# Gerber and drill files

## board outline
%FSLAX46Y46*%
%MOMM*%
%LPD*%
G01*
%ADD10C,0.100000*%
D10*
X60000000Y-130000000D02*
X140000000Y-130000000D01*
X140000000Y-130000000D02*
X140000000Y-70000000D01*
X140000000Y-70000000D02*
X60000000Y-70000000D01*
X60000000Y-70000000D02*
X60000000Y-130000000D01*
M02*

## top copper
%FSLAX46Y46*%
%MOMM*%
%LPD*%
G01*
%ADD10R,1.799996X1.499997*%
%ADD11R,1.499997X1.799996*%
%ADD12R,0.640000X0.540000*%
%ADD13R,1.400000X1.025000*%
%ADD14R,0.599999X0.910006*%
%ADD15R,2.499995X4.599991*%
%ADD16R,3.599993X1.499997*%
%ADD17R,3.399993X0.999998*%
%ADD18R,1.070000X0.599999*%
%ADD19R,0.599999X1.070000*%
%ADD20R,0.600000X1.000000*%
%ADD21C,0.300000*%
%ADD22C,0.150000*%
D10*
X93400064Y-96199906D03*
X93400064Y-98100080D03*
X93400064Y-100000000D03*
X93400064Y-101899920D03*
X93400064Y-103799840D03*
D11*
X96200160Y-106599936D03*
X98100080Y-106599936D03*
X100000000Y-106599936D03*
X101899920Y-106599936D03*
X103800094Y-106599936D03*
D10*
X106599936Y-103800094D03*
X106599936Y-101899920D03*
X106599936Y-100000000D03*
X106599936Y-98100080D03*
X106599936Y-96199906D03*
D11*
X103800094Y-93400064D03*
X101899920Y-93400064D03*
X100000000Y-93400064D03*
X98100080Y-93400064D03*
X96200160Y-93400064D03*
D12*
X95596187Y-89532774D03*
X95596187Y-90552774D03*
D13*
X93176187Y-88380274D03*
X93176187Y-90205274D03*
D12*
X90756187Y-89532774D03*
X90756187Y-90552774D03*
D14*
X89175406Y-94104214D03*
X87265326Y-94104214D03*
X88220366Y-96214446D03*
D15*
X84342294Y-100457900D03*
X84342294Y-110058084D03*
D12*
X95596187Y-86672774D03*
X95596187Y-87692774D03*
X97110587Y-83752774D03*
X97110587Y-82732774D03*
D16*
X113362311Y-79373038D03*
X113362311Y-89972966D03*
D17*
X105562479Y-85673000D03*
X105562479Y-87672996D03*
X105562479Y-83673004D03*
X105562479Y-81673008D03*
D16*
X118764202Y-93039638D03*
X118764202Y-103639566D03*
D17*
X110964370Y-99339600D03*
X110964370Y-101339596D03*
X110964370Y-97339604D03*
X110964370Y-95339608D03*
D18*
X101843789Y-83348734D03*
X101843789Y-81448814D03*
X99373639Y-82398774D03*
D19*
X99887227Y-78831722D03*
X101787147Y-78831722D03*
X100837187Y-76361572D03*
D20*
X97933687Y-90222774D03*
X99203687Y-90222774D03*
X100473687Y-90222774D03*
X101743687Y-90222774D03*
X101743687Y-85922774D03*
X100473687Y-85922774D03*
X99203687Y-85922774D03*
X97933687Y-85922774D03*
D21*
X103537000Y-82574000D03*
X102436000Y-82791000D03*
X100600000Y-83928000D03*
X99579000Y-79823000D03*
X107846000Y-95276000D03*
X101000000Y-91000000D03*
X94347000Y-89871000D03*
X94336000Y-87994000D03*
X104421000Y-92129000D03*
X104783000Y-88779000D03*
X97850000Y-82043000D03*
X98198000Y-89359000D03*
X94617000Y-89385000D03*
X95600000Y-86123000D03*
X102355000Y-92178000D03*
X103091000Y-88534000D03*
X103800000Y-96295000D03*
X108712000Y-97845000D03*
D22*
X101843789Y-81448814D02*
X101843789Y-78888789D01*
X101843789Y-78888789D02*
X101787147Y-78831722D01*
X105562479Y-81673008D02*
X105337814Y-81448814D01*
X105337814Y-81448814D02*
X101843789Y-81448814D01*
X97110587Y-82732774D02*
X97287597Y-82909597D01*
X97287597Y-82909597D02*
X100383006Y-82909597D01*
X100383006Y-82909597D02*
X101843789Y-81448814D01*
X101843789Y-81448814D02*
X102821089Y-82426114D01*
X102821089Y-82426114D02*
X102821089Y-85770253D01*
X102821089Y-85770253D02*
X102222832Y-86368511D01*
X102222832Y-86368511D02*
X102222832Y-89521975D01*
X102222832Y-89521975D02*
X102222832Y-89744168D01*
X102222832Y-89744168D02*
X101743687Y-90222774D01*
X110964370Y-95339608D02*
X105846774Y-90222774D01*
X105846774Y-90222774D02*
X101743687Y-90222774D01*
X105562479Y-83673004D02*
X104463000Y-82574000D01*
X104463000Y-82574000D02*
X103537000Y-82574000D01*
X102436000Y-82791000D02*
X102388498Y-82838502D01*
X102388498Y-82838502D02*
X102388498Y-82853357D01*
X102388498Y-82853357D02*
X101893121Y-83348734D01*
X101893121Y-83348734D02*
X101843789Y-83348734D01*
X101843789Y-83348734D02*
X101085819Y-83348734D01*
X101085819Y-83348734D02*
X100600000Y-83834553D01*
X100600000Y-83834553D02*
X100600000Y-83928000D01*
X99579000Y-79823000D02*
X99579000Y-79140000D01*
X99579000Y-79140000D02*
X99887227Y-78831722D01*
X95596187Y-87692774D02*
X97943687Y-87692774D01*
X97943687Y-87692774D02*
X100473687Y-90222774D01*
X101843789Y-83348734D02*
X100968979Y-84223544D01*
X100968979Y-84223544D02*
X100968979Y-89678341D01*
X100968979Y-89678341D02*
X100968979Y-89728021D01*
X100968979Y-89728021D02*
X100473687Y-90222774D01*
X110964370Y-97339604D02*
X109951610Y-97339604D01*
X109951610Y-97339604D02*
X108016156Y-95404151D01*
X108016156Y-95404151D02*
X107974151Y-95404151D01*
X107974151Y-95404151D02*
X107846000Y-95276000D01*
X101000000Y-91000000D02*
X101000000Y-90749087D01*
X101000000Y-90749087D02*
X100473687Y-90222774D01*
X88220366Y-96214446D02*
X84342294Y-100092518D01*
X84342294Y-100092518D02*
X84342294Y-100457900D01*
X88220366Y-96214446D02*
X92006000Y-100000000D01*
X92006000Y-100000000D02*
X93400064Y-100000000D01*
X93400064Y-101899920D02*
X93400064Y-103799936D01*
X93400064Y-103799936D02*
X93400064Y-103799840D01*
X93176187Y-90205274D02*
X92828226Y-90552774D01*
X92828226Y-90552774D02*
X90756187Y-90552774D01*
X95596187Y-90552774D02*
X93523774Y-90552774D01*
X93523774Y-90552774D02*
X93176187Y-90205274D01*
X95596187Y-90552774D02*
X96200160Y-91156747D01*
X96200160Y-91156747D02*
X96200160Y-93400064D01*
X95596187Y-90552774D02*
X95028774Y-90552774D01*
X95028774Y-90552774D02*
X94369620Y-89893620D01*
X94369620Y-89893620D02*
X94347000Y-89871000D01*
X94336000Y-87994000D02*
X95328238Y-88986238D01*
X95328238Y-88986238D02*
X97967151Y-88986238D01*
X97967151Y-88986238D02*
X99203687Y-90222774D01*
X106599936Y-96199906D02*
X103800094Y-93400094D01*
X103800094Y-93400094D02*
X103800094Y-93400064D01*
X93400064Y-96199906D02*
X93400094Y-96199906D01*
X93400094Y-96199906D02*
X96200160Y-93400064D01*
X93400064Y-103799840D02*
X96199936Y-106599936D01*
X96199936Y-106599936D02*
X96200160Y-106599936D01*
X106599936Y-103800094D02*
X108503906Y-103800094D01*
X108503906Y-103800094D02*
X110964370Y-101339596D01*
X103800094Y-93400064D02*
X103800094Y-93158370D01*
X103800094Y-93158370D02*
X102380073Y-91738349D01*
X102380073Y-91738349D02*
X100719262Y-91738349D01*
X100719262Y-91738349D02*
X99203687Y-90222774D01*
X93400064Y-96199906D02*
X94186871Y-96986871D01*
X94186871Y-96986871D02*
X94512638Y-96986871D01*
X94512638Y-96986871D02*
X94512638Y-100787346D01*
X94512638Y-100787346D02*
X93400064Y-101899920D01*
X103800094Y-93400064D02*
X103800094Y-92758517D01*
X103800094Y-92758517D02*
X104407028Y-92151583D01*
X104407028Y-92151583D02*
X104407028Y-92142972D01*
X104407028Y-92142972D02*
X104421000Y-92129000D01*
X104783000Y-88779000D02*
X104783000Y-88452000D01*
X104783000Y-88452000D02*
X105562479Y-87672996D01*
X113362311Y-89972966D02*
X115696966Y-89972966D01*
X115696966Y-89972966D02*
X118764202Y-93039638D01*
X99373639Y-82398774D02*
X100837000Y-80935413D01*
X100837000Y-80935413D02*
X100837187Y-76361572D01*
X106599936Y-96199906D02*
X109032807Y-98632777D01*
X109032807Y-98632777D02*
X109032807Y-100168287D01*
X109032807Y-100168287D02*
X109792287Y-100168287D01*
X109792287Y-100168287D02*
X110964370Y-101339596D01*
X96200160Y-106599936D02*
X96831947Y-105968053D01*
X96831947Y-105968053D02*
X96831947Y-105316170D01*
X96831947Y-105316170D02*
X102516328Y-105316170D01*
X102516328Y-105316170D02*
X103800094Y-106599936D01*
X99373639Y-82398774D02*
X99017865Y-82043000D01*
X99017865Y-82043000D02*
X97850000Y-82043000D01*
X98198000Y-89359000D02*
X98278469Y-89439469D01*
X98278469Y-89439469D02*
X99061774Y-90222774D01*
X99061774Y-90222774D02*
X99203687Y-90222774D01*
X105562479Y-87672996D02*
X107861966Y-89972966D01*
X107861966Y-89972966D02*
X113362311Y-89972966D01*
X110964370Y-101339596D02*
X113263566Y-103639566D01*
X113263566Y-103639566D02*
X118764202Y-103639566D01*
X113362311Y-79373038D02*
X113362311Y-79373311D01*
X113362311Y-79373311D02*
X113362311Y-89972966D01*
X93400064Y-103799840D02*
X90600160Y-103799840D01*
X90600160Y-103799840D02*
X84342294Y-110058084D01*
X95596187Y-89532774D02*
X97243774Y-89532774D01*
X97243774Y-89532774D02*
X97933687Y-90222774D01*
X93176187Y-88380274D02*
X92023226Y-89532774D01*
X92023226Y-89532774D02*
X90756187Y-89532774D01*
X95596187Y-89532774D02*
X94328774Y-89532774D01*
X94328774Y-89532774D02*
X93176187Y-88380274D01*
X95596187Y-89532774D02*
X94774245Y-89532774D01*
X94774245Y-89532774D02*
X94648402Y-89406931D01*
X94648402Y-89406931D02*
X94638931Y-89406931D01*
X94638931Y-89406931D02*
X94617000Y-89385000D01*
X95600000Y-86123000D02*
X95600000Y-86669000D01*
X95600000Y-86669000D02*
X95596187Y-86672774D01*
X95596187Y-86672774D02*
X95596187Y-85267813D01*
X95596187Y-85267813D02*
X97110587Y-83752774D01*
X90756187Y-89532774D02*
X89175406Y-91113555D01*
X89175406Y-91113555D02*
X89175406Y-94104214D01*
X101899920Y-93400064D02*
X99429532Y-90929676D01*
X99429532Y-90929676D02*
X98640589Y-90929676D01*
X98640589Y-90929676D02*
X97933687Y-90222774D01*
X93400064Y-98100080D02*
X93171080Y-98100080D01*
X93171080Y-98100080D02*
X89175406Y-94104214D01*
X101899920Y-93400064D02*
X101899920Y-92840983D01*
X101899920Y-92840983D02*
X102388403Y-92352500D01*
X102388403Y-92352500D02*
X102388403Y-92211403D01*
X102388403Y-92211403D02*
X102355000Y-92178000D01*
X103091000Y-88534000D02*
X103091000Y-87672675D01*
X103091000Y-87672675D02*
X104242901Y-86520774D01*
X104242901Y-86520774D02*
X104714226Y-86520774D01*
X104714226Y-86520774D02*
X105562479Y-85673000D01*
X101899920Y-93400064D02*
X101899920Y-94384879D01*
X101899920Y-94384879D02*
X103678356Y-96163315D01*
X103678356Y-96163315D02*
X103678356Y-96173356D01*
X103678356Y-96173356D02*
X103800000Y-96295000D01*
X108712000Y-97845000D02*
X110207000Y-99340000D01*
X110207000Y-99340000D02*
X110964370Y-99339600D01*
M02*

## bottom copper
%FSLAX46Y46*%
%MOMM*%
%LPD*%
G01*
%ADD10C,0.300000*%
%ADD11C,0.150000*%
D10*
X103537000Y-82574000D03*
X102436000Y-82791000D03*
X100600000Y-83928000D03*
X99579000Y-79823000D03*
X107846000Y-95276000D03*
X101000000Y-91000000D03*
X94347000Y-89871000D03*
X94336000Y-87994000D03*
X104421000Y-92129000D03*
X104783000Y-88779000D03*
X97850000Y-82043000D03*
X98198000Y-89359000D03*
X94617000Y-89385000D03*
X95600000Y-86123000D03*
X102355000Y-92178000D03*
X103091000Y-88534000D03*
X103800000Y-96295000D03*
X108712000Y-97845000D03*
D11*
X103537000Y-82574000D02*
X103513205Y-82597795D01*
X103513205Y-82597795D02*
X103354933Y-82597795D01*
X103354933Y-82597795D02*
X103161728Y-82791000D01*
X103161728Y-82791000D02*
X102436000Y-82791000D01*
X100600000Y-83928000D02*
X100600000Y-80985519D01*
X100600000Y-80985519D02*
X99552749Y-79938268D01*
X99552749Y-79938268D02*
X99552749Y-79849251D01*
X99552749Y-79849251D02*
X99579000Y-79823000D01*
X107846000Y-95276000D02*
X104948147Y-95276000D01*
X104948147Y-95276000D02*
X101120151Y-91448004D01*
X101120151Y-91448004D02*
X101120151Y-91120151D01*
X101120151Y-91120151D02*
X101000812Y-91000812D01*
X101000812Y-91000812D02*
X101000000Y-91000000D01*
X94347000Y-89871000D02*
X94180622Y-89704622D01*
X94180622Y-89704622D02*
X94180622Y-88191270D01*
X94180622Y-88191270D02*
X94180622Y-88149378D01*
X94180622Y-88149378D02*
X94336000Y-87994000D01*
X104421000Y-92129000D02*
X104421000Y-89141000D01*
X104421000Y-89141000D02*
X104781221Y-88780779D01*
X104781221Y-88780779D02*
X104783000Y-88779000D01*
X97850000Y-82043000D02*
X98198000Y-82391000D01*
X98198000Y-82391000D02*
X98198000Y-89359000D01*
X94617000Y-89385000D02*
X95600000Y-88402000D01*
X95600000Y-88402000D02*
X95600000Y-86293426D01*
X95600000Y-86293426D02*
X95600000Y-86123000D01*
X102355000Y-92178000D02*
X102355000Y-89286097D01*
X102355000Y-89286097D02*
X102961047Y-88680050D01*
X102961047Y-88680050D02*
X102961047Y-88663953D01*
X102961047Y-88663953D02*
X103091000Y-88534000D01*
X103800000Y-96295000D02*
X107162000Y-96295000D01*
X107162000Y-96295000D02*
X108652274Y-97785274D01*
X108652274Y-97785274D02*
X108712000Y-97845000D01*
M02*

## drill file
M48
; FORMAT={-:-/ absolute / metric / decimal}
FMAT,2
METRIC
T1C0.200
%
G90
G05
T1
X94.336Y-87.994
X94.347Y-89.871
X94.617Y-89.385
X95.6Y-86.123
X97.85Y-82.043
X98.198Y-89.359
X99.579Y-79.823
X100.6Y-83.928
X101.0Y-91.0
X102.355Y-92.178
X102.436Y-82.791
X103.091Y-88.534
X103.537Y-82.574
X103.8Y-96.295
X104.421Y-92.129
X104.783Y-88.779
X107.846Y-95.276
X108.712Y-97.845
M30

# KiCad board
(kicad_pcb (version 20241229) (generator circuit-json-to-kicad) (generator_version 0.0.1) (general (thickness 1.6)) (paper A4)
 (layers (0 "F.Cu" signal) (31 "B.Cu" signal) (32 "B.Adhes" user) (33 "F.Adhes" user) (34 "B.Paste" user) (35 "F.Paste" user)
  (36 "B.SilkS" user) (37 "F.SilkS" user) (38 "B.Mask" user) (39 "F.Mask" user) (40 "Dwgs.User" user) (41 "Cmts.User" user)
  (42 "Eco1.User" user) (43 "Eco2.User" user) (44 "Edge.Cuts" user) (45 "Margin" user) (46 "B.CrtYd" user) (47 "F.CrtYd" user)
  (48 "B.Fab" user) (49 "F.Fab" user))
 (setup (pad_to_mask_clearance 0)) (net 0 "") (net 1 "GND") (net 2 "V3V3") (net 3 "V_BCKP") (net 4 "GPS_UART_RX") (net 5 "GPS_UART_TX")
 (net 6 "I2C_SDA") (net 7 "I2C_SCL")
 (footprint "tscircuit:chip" (layer F.Cu) (at 100 100 0)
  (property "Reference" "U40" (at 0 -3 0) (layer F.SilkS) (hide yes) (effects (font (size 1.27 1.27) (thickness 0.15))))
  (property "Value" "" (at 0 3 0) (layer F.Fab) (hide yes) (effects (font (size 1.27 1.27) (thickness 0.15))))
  (pad "1" smd rect (at -6.5999360000001275 -3.8000939999998877 0) (size 1.7999964 1.499997) (layers F.Cu F.Paste F.Mask) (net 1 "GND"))
  (pad "2" smd rect (at -6.5999360000001275 -1.899919999999895 0) (size 1.7999964 1.499997) (layers F.Cu F.Paste F.Mask) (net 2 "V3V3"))
  (pad "3" smd rect (at -6.5999360000001275 5.684341886080802e-14 0) (size 1.7999964 1.499997) (layers F.Cu F.Paste F.Mask) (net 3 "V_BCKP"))
  (pad "4" smd rect (at -6.5999360000001275 1.8999200000000087 0) (size 1.7999964 1.499997) (layers F.Cu F.Paste F.Mask) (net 1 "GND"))
  (pad "5" smd rect (at -6.5999360000001275 3.7998400000000743 0) (size 1.7999964 1.499997) (layers F.Cu F.Paste F.Mask) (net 1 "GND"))
  (pad "6" smd rect (at -3.7998399999999606 6.599936000000014 0) (size 1.499997 1.7999964) (layers F.Cu F.Paste F.Mask) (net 1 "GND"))
  (pad "7" smd rect (at -1.899919999999895 6.599936000000014 0) (size 1.499997 1.7999964) (layers F.Cu F.Paste F.Mask))
  (pad "8" smd rect (at -5.684341886080802e-14 6.599936000000014 0) (size 1.499997 1.7999964) (layers F.Cu F.Paste F.Mask))
  (pad "9" smd rect (at 1.899919999999895 6.599936000000014 0) (size 1.499997 1.7999964) (layers F.Cu F.Paste F.Mask))
  (pad "10" smd rect (at 3.8000940000000014 6.599936000000014 0) (size 1.499997 1.7999964) (layers F.Cu F.Paste F.Mask) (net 1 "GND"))
  (pad "11" smd rect (at 6.5999360000001275 3.800094000000115 0) (size 1.7999964 1.499997) (layers F.Cu F.Paste F.Mask) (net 1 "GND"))
  (pad "12" smd rect (at 6.5999360000001275 1.8999200000000087 0) (size 1.7999964 1.499997) (layers F.Cu F.Paste F.Mask))
  (pad "13" smd rect (at 6.5999360000001275 5.684341886080802e-14 0) (size 1.7999964 1.499997) (layers F.Cu F.Paste F.Mask)
   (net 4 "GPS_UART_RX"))
  (pad "14" smd rect (at 6.5999360000001275 -1.899919999999895 0) (size 1.7999964 1.499997) (layers F.Cu F.Paste F.Mask)
   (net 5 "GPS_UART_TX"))
  (pad "15" smd rect (at 6.5999360000001275 -3.8000939999998877 0) (size 1.7999964 1.499997) (layers F.Cu F.Paste F.Mask) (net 1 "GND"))
  (pad "16" smd rect (at 3.8000940000000014 -6.599936000000014 0) (size 1.499997 1.7999964) (layers F.Cu F.Paste F.Mask) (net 1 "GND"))
  (pad "17" smd rect (at 1.899919999999895 -6.599936000000014 0) (size 1.499997 1.7999964) (layers F.Cu F.Paste F.Mask) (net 2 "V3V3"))
  (pad "18" smd rect (at -5.684341886080802e-14 -6.599936000000014 0) (size 1.499997 1.7999964) (layers F.Cu F.Paste F.Mask))
  (pad "19" smd rect (at -1.899919999999895 -6.599936000000014 0) (size 1.499997 1.7999964) (layers F.Cu F.Paste F.Mask))
  (pad "20" smd rect (at -3.7998399999999606 -6.599936000000014 0) (size 1.499997 1.7999964) (layers F.Cu F.Paste F.Mask) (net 1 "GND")))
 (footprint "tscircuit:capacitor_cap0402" (layer F.Cu) (at 95.59618690909089 90.04277400000001 -90.00000000000001)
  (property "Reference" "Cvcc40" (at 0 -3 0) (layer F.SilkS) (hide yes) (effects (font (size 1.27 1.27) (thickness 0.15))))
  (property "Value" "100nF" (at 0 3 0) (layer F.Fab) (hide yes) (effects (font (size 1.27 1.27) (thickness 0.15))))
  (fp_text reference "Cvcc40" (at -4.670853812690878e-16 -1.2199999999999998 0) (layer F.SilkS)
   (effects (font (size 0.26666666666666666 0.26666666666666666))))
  (pad "1" smd rect (at -0.5099999999999998 8.881784197001252e-16 0) (size 0.64 0.54) (layers F.Cu F.Paste F.Mask) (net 2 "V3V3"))
  (pad "2" smd rect (at 0.5099999999999998 0 0) (size 0.64 0.54) (layers F.Cu F.Paste F.Mask) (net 1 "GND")))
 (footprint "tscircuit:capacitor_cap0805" (layer F.Cu) (at 93.17618690909089 89.29277400000001 -90.00000000000001)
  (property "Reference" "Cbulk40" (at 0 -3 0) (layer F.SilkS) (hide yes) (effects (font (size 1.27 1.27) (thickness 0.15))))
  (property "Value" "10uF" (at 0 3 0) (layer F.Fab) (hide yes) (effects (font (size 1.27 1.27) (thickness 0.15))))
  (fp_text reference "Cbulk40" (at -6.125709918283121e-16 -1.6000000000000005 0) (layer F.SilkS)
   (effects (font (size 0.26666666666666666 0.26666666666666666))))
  (pad "1" smd rect (at -0.9124999999999996 0 0) (size 1.4 1.025) (layers F.Cu F.Paste F.Mask) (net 2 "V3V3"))
  (pad "2" smd rect (at 0.9124999999999996 -8.881784197001252e-16 0) (size 1.4 1.025) (layers F.Cu F.Paste F.Mask) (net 1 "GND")))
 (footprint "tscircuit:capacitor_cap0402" (layer F.Cu) (at 90.75618690909089 90.04277400000001 -90.00000000000001)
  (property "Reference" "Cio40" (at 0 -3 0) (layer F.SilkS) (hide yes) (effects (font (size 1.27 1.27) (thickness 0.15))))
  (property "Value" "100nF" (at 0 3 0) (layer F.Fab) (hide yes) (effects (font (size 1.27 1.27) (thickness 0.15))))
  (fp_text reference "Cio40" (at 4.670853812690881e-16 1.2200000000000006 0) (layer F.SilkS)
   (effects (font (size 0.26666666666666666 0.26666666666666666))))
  (pad "1" smd rect (at -0.5099999999999998 0 0) (size 0.64 0.54) (layers F.Cu F.Paste F.Mask) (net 2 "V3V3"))
  (pad "2" smd rect (at 0.5099999999999998 0 0) (size 0.64 0.54) (layers F.Cu F.Paste F.Mask) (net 1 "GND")))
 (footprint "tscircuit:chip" (layer F.Cu) (at 88.22036600000001 95.15933033333334 90)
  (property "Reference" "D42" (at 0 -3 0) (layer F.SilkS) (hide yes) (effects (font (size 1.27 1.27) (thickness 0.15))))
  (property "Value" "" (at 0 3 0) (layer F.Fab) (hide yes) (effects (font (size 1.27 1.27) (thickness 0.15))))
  (pad "1" smd rect (at 1.0551160000000053 0.9550400000000039 0) (size 0.5999987999999999 0.9100057999999999) (layers F.Cu F.Paste F.Mask)
   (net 2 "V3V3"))
  (pad "2" smd rect (at 1.0551160000000053 -0.9550400000000039 0) (size 0.5999987999999999 0.9100057999999999) (layers F.Cu F.Paste F.Mask))
  (pad "3" smd rect (at -1.0551160000000053 7.105427357601002e-15 0) (size 0.5999987999999999 0.9100057999999999)
   (layers F.Cu F.Paste F.Mask) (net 3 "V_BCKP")))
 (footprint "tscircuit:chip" (layer F.Cu) (at 84.34229399999987 105.25799233333349 -90.00000000000001)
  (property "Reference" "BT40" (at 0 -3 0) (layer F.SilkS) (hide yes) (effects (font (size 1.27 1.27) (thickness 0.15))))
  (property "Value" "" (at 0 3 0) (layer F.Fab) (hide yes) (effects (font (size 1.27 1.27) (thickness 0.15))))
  (pad "1" smd rect (at -4.80009200000012 1.7763568394002505e-15 0) (size 2.4999949999999997 4.5999908) (layers F.Cu F.Paste F.Mask)
   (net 3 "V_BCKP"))
  (pad "2" smd rect (at 4.800092000000118 -1.7763568394002505e-15 0) (size 2.4999949999999997 4.5999908) (layers F.Cu F.Paste F.Mask)
   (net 1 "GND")))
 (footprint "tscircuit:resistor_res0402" (layer F.Cu) (at 95.59618690909089 87.18277400000002 -90.00000000000001)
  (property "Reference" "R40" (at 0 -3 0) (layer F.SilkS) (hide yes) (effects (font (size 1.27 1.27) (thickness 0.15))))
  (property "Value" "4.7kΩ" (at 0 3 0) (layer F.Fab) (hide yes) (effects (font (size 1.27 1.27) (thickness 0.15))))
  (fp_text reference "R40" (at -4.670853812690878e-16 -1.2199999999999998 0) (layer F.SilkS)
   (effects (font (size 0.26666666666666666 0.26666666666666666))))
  (pad "1" smd rect (at -0.5099999999999998 0 0) (size 0.64 0.54) (layers F.Cu F.Paste F.Mask) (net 2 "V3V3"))
  (pad "2" smd rect (at 0.5099999999999998 -8.881784197001252e-16 0) (size 0.64 0.54) (layers F.Cu F.Paste F.Mask) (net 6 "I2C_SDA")))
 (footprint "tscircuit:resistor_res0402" (layer F.Cu) (at 97.11058690909073 83.24277400000001 90)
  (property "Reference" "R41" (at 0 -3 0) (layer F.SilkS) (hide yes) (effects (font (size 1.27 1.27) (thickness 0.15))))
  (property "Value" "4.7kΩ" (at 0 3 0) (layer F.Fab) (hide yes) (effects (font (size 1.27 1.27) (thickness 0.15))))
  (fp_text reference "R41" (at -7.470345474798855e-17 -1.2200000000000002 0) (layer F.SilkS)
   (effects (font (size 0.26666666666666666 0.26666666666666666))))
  (pad "1" smd rect (at -0.5100000000000016 0 0) (size 0.64 0.54) (layers F.Cu F.Paste F.Mask) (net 2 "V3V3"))
  (pad "2" smd rect (at 0.5100000000000016 0 0) (size 0.64 0.54) (layers F.Cu F.Paste F.Mask) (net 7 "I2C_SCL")))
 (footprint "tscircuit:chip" (layer F.Cu) (at 109.51239480909098 84.673002 90)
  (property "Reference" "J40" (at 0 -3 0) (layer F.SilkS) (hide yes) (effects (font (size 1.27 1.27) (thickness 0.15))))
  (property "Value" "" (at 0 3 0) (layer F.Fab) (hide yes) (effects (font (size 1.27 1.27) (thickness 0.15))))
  (pad "5" smd rect (at 5.299963999999989 3.8499161000000193 0) (size 3.5999928 1.499997) (layers F.Cu F.Paste F.Mask) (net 1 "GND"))
  (pad "6" smd rect (at -5.299963999999989 3.849916100000021 0) (size 3.5999928 1.499997) (layers F.Cu F.Paste F.Mask) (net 1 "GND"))
  (pad "2" smd rect (at -0.9999979999999482 -3.9499159000000175 0) (size 3.3999932 0.9999979999999999) (layers F.Cu F.Paste F.Mask)
   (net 2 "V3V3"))
  (pad "1" smd rect (at -2.999994000000072 -3.9499159000000175 0) (size 3.3999932 0.9999979999999999) (layers F.Cu F.Paste F.Mask)
   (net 1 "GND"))
  (pad "3" smd rect (at 0.9999979999999482 -3.9499159000000175 0) (size 3.3999932 0.9999979999999999) (layers F.Cu F.Paste F.Mask)
   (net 6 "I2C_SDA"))
  (pad "4" smd rect (at 2.9999939999999583 -3.9499159000000175 0) (size 3.3999932 0.9999979999999999) (layers F.Cu F.Paste F.Mask)
   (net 7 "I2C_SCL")))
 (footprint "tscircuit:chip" (layer F.Cu) (at 114.9142860999999 98.33960200000001 90)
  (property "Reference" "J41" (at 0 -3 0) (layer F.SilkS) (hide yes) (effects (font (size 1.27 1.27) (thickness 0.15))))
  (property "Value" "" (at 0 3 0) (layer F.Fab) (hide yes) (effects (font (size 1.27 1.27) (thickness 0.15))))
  (pad "5" smd rect (at 5.299963999999989 3.8499161000000193 0) (size 3.5999928 1.499997) (layers F.Cu F.Paste F.Mask) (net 1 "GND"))
  (pad "6" smd rect (at -5.299963999999989 3.8499161000000193 0) (size 3.5999928 1.499997) (layers F.Cu F.Paste F.Mask) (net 1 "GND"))
  (pad "2" smd rect (at -0.9999979999999482 -3.9499159000000184 0) (size 3.3999932 0.9999979999999999) (layers F.Cu F.Paste F.Mask)
   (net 2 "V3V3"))
  (pad "1" smd rect (at -2.999994000000072 -3.9499159000000184 0) (size 3.3999932 0.9999979999999999) (layers F.Cu F.Paste F.Mask)
   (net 1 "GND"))
  (pad "3" smd rect (at 0.9999979999999482 -3.9499159000000184 0) (size 3.3999932 0.9999979999999999) (layers F.Cu F.Paste F.Mask)
   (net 6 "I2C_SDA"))
  (pad "4" smd rect (at 2.9999939999999583 -3.9499159000000184 0) (size 3.3999932 0.9999979999999999) (layers F.Cu F.Paste F.Mask)
   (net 7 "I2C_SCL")))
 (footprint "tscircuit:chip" (layer F.Cu) (at 100.60871390909071 82.39877400000002 0)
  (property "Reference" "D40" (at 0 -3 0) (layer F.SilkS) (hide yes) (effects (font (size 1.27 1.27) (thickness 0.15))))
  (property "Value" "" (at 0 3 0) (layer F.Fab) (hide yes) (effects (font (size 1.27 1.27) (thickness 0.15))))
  (pad "1" smd rect (at 1.2350749999999948 0.9499599999999191 0) (size 1.0700004 0.5999987999999999) (layers F.Cu F.Paste F.Mask)
   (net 6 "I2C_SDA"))
  (pad "2" smd rect (at 1.2350749999999948 -0.9499599999999191 0) (size 1.0700004 0.5999987999999999) (layers F.Cu F.Paste F.Mask)
   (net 7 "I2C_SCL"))
  (pad "3" smd rect (at -1.2350749999999948 0 0) (size 1.0700004 0.5999987999999999) (layers F.Cu F.Paste F.Mask) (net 1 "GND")))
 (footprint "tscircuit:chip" (layer F.Cu) (at 100.83718690909089 77.59664700000003 -90.00000000000001)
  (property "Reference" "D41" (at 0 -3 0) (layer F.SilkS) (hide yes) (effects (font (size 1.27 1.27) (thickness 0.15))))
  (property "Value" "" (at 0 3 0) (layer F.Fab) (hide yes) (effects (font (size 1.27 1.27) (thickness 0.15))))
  (pad "1" smd rect (at 1.2350749999999948 0.9499599999999189 0) (size 0.5999987999999999 1.0700004) (layers F.Cu F.Paste F.Mask)
   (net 6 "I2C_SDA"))
  (pad "2" smd rect (at 1.2350749999999948 -0.9499599999999194 0) (size 0.5999987999999999 1.0700004) (layers F.Cu F.Paste F.Mask)
   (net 7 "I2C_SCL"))
  (pad "3" smd rect (at -1.2350749999999948 3.3306690738754696e-16 0) (size 0.5999987999999999 1.0700004) (layers F.Cu F.Paste F.Mask)
   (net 1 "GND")))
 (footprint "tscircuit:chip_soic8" (layer F.Cu) (at 99.83868690909088 88.07277400000001 90)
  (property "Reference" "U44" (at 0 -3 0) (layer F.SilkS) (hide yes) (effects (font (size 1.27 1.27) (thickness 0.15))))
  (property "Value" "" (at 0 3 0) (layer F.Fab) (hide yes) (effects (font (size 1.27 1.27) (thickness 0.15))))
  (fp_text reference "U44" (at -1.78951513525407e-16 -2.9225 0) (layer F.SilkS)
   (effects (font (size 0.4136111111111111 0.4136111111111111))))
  (pad "1" smd rect (at -2.1500000000000004 -1.905 0) (size 0.6 1) (layers F.Cu F.Paste F.Mask) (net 2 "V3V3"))
  (pad "2" smd rect (at -2.1500000000000004 -0.635 0) (size 0.6 1) (layers F.Cu F.Paste F.Mask) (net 1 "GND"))
  (pad "3" smd rect (at -2.1500000000000004 0.635 0) (size 0.6 1) (layers F.Cu F.Paste F.Mask) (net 6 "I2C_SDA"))
  (pad "4" smd rect (at -2.1500000000000004 1.9049999999999998 0) (size 0.6 1) (layers F.Cu F.Paste F.Mask) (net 7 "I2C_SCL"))
  (pad "5" smd rect (at 2.1500000000000004 1.905 0) (size 0.6 1) (layers F.Cu F.Paste F.Mask))
  (pad "6" smd rect (at 2.1500000000000004 0.635 0) (size 0.6 1) (layers F.Cu F.Paste F.Mask))
  (pad "7" smd rect (at 2.1500000000000004 -0.635 0) (size 0.6 1) (layers F.Cu F.Paste F.Mask))
  (pad "8" smd rect (at 2.1500000000000004 -1.905 0) (size 0.6 1) (layers F.Cu F.Paste F.Mask)))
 (segment (start 101.8437889090907 81.4488140000001) (end 101.8437889090907 78.8887889090907) (width 0.15) (layer F.Cu) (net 7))
 (segment (start 101.8437889090907 78.8887889090907) (end 101.78714690909081 78.83172200000003) (width 0.15) (layer F.Cu) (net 7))
 (segment (start 105.56247890909097 81.67300800000004) (end 105.3378140000001 81.4488140000001) (width 0.15) (layer F.Cu) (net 7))
 (segment (start 105.3378140000001 81.4488140000001) (end 101.8437889090907 81.4488140000001) (width 0.15) (layer F.Cu) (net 7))
 (segment (start 97.11058690909073 82.732774) (end 97.28759723607489 82.90959723607489) (width 0.15) (layer F.Cu) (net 7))
 (segment (start 97.28759723607489 82.90959723607489) (end 100.3830056730159 82.90959723607489) (width 0.15) (layer F.Cu) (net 7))
 (segment (start 100.3830056730159 82.90959723607489) (end 101.8437889090907 81.4488140000001) (width 0.15) (layer F.Cu) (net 7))
 (segment (start 101.8437889090907 81.4488140000001) (end 102.82108920157091 82.4261142924803) (width 0.15) (layer F.Cu) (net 7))
 (segment (start 102.82108920157091 82.4261142924803) (end 102.82108920157091 85.77025333037076) (width 0.15) (layer F.Cu) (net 7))
 (segment (start 102.82108920157091 85.77025333037076) (end 102.22283199472146 86.3685105372202) (width 0.15) (layer F.Cu) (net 7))
 (segment (start 102.22283199472146 86.3685105372202) (end 102.22283199472146 89.52197478346525) (width 0.15) (layer F.Cu) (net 7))
 (segment (start 102.22283199472146 89.52197478346525) (end 102.22283199472146 89.74416800527854) (width 0.15) (layer F.Cu) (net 7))
 (segment (start 102.22283199472146 89.74416800527854) (end 101.74368690909088 90.22277400000002) (width 0.15) (layer F.Cu) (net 7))
 (segment (start 110.96437019999988 95.33960800000006) (end 105.84677400000001 90.22277400000002) (width 0.15) (layer F.Cu) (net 7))
 (segment (start 105.84677400000001 90.22277400000002) (end 101.74368690909088 90.22277400000002) (width 0.15) (layer F.Cu) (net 7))
 (segment (start 105.56247890909097 83.67300400000005) (end 104.46300000000001 82.574) (width 0.15) (layer F.Cu) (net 6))
 (segment (start 104.46300000000001 82.574) (end 103.537 82.574) (width 0.15) (layer F.Cu) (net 6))
 (segment (start 103.537 82.574) (end 103.51320467501183 82.59779532498817) (width 0.15) (layer B.Cu) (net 6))
 (segment (start 103.51320467501183 82.59779532498817) (end 103.35493272030583 82.59779532498817) (width 0.15) (layer B.Cu) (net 6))
 (segment (start 103.35493272030583 82.59779532498817) (end 103.161728045294 82.791) (width 0.15) (layer B.Cu) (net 6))
 (segment (start 103.161728045294 82.791) (end 102.436 82.791) (width 0.15) (layer B.Cu) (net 6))
 (segment (start 102.436 82.791) (end 102.38849819781895 82.83850180218104) (width 0.15) (layer F.Cu) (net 6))
 (segment (start 102.38849819781895 82.83850180218104) (end 102.38849819781895 82.85335684220804) (width 0.15) (layer F.Cu) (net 6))
 (segment (start 102.38849819781895 82.85335684220804) (end 101.89312104002707 83.34873399999994) (width 0.15) (layer F.Cu) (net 6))
 (segment (start 101.89312104002707 83.34873399999994) (end 101.8437889090907 83.34873399999994) (width 0.15) (layer F.Cu) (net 6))
 (segment (start 101.8437889090907 83.34873399999994) (end 101.08581889302985 83.34873399999994) (width 0.15) (layer F.Cu) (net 6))
 (segment (start 101.08581889302985 83.34873399999994) (end 100.6 83.8345528930298) (width 0.15) (layer F.Cu) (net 6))
 (segment (start 100.6 83.8345528930298) (end 100.6 83.928) (width 0.15) (layer F.Cu) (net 6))
 (segment (start 100.6 83.928) (end 100.6 80.98551869050203) (width 0.15) (layer B.Cu) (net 6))
 (segment (start 100.6 80.98551869050203) (end 99.55274927718217 79.9382679676842) (width 0.15) (layer B.Cu) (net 6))
 (segment (start 99.55274927718217 79.9382679676842) (end 99.55274927718217 79.84925072281783) (width 0.15) (layer B.Cu) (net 6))
 (segment (start 99.55274927718217 79.84925072281783) (end 99.579 79.82300000000001) (width 0.15) (layer B.Cu) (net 6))
 (segment (start 99.579 79.82300000000001) (end 99.579 79.14) (width 0.15) (layer F.Cu) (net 6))
 (segment (start 99.579 79.14) (end 99.88722690909097 78.83172200000003) (width 0.15) (layer F.Cu) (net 6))
 (segment (start 95.59618690909089 87.69277400000001) (end 97.94368690909089 87.69277400000001) (width 0.15) (layer F.Cu) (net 6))
 (segment (start 97.94368690909089 87.69277400000001) (end 100.47368690909089 90.22277400000002) (width 0.15) (layer F.Cu) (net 6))
 (segment (start 101.8437889090907 83.34873399999994) (end 100.96897882086891 84.22354408822173) (width 0.15) (layer F.Cu) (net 6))
 (segment (start 100.96897882086891 84.22354408822173) (end 100.96897882086891 89.6783406450725) (width 0.15) (layer F.Cu) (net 6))
 (segment (start 100.96897882086891 89.6783406450725) (end 100.96897882086891 89.72802117913109) (width 0.15) (layer F.Cu) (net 6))
 (segment (start 100.96897882086891 89.72802117913109) (end 100.47368690909089 90.22277400000002) (width 0.15) (layer F.Cu) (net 6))
 (segment (start 110.96437019999988 97.33960400000007) (end 109.95160956777949 97.33960400000007) (width 0.15) (layer F.Cu) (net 6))
 (segment (start 109.95160956777949 97.33960400000007) (end 108.0161560686697 95.4041505008903) (width 0.15) (layer F.Cu) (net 6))
 (segment (start 108.0161560686697 95.4041505008903) (end 107.97415050089029 95.4041505008903) (width 0.15) (layer F.Cu) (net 6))
 (segment (start 107.97415050089029 95.4041505008903) (end 107.846 95.276) (width 0.15) (layer F.Cu) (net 6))
 (segment (start 107.846 95.276) (end 104.94814723394575 95.276) (width 0.15) (layer B.Cu) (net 6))
 (segment (start 104.94814723394575 95.276) (end 101.12015121683972 91.44800398289397) (width 0.15) (layer B.Cu) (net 6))
 (segment (start 101.12015121683972 91.44800398289397) (end 101.12015121683972 91.12015121683972) (width 0.15) (layer B.Cu) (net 6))
 (segment (start 101.12015121683972 91.12015121683972) (end 101.00081204914446 91.00081204914446) (width 0.15) (layer B.Cu) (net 6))
 (segment (start 101.00081204914446 91.00081204914446) (end 101 91) (width 0.15) (layer B.Cu) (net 6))
 (segment (start 101 91) (end 101 90.74908709090913) (width 0.15) (layer F.Cu) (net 6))
 (segment (start 101 90.74908709090913) (end 100.47368690909089 90.22277400000002) (width 0.15) (layer F.Cu) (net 6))
 (segment (start 88.22036600000003 96.21444633333336) (end 84.34229399999987 100.09251833333352) (width 0.15) (layer F.Cu) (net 3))
 (segment (start 84.34229399999987 100.09251833333352) (end 84.34229399999987 100.45790033333337) (width 0.15) (layer F.Cu) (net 3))
 (segment (start 88.22036600000003 96.21444633333336) (end 92.00600000000006 100.00000000000006) (width 0.15) (layer F.Cu) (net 3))
 (segment (start 92.00600000000006 100.00000000000006) (end 93.40006399999987 100.00000000000006) (width 0.15) (layer F.Cu) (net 3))
 (segment (start 93.40006399999987 101.89992000000001) (end 93.40006399999987 103.79993600000013) (width 0.15) (layer F.Cu) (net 1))
 (segment (start 93.40006399999987 103.79993600000013) (end 93.40006399999987 103.79984000000007) (width 0.15) (layer F.Cu) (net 1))
 (segment (start 93.17618690909089 90.20527400000002) (end 92.82822599999999 90.55277400000001) (width 0.15) (layer F.Cu) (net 1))
 (segment (start 92.82822599999999 90.55277400000001) (end 90.75618690909089 90.55277400000001) (width 0.15) (layer F.Cu) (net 1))
 (segment (start 95.59618690909089 90.55277400000001) (end 93.52377400000002 90.55277400000001) (width 0.15) (layer F.Cu) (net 1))
 (segment (start 93.52377400000002 90.55277400000001) (end 93.17618690909089 90.20527400000002) (width 0.15) (layer F.Cu) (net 1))
 (segment (start 95.59618690909089 90.55277400000001) (end 96.20016000000004 91.15674709090916) (width 0.15) (layer F.Cu) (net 1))
 (segment (start 96.20016000000004 91.15674709090916) (end 96.20016000000004 93.40006399999999) (width 0.15) (layer F.Cu) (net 1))
 (segment (start 95.59618690909089 90.55277400000001) (end 95.02877400000001 90.55277400000001) (width 0.15) (layer F.Cu) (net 1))
 (segment (start 95.02877400000001 90.55277400000001) (end 94.36961983876657 89.89361983876657) (width 0.15) (layer F.Cu) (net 1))
 (segment (start 94.36961983876657 89.89361983876657) (end 94.347 89.871) (width 0.15) (layer F.Cu) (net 1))
 (segment (start 94.347 89.871) (end 94.18062236750478 89.70462236750478) (width 0.15) (layer B.Cu) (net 1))
 (segment (start 94.18062236750478 89.70462236750478) (end 94.18062236750478 88.19127003402869) (width 0.15) (layer B.Cu) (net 1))
 (segment (start 94.18062236750478 88.19127003402869) (end 94.18062236750478 88.14937763249523) (width 0.15) (layer B.Cu) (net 1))
 (segment (start 94.18062236750478 88.14937763249523) (end 94.336 87.994) (width 0.15) (layer B.Cu) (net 1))
 (segment (start 94.336 87.994) (end 95.32823791632767 88.98623791632767) (width 0.15) (layer F.Cu) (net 1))
 (segment (start 95.32823791632767 88.98623791632767) (end 97.96715082541853 88.98623791632767) (width 0.15) (layer F.Cu) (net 1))
 (segment (start 97.96715082541853 88.98623791632767) (end 99.20368690909089 90.22277400000002) (width 0.15) (layer F.Cu) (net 1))
 (segment (start 106.59993600000013 96.19990600000011) (end 103.800094 93.400094) (width 0.15) (layer F.Cu) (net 1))
 (segment (start 103.800094 93.400094) (end 103.800094 93.40006399999999) (width 0.15) (layer F.Cu) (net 1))
 (segment (start 93.40006399999987 96.19990600000011) (end 93.40009399999988 96.19990600000011) (width 0.15) (layer F.Cu) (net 1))
 (segment (start 93.40009399999988 96.19990600000011) (end 96.20016000000004 93.40006399999999) (width 0.15) (layer F.Cu) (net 1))
 (segment (start 93.40006399999987 103.79984000000007) (end 96.19993600000001 106.59993600000001) (width 0.15) (layer F.Cu) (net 1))
 (segment (start 96.19993600000001 106.59993600000001) (end 96.20016000000004 106.59993600000001) (width 0.15) (layer F.Cu) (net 1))
 (segment (start 106.59993600000013 103.80009400000012) (end 108.50390599999989 103.80009400000012) (width 0.15) (layer F.Cu) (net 1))
 (segment (start 108.50390599999989 103.80009400000012) (end 110.96437019999988 101.33959600000009) (width 0.15) (layer F.Cu) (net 1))
 (segment (start 103.800094 93.40006399999999) (end 103.800094 93.15836968972701) (width 0.15) (layer F.Cu) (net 1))
 (segment (start 103.800094 93.15836968972701) (end 102.3800734252521 91.7383491149791) (width 0.15) (layer F.Cu) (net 1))
 (segment (start 102.3800734252521 91.7383491149791) (end 100.71926202406998 91.7383491149791) (width 0.15) (layer F.Cu) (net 1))
 (segment (start 100.71926202406998 91.7383491149791) (end 99.20368690909089 90.22277400000002) (width 0.15) (layer F.Cu) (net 1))
 (segment (start 93.40006399999987 96.19990600000011) (end 94.18687091737846 96.98687091737845) (width 0.15) (layer F.Cu) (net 1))
 (segment (start 94.18687091737846 96.98687091737845) (end 94.51263838721975 96.98687091737845) (width 0.15) (layer F.Cu) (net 1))
 (segment (start 94.51263838721975 96.98687091737845) (end 94.51263838721975 100.78734561278013) (width 0.15) (layer F.Cu) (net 1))
 (segment (start 94.51263838721975 100.78734561278013) (end 93.40006399999987 101.89992000000001) (width 0.15) (layer F.Cu) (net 1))
 (segment (start 103.800094 93.40006399999999) (end 103.800094 92.75851721283978) (width 0.15) (layer F.Cu) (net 1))
 (segment (start 103.800094 92.75851721283978) (end 104.40702837633002 92.15158283650976) (width 0.15) (layer F.Cu) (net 1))
 (segment (start 104.40702837633002 92.15158283650976) (end 104.40702837633002 92.14297162366998) (width 0.15) (layer F.Cu) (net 1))
 (segment (start 104.40702837633002 92.14297162366998) (end 104.421 92.129) (width 0.15) (layer F.Cu) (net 1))
 (segment (start 104.421 92.129) (end 104.421 89.141) (width 0.15) (layer B.Cu) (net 1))
 (segment (start 104.421 89.141) (end 104.78122118328378 88.78077881671624) (width 0.15) (layer B.Cu) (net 1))
 (segment (start 104.78122118328378 88.78077881671624) (end 104.783 88.779) (width 0.15) (layer B.Cu) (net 1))
 (segment (start 104.783 88.779) (end 104.783 88.452) (width 0.15) (layer F.Cu) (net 1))
 (segment (start 104.783 88.452) (end 105.56247890909097 87.67299600000007) (width 0.15) (layer F.Cu) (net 1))
 (segment (start 113.36231090909101 89.97296599999999) (end 115.69696599999999 89.97296599999999) (width 0.15) (layer F.Cu) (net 1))
 (segment (start 115.69696599999999 89.97296599999999) (end 118.76420219999991 93.03963800000002) (width 0.15) (layer F.Cu) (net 1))
 (segment (start 99.37363890909072 82.39877400000002) (end 100.837 80.93541290909073) (width 0.15) (layer F.Cu) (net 1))
 (segment (start 100.837 80.93541290909073) (end 100.83718690909089 76.36157200000004) (width 0.15) (layer F.Cu) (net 1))
 (segment (start 106.59993600000013 96.19990600000011) (end 109.03280716384539 98.63277716384538) (width 0.15) (layer F.Cu) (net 1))
 (segment (start 109.03280716384539 98.63277716384538) (end 109.03280716384539 100.16828745876474) (width 0.15) (layer F.Cu) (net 1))
 (segment (start 109.03280716384539 100.16828745876474) (end 109.79228745876475 100.16828745876474) (width 0.15) (layer F.Cu) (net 1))
 (segment (start 109.79228745876475 100.16828745876474) (end 110.96437019999988 101.33959600000009) (width 0.15) (layer F.Cu) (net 1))
 (segment (start 96.20016000000004 106.59993600000001) (end 96.83194656006272 105.96805343993728) (width 0.15) (layer F.Cu) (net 1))
 (segment (start 96.83194656006272 105.96805343993728) (end 96.83194656006272 105.31617044019791) (width 0.15) (layer F.Cu) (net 1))
 (segment (start 96.83194656006272 105.31617044019791) (end 102.5163284401979 105.31617044019791) (width 0.15) (layer F.Cu) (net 1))
 (segment (start 102.5163284401979 105.31617044019791) (end 103.800094 106.59993600000001) (width 0.15) (layer F.Cu) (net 1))
 (segment (start 99.37363890909072 82.39877400000002) (end 99.01786490909069 82.043) (width 0.15) (layer F.Cu) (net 1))
 (segment (start 99.01786490909069 82.043) (end 97.85 82.043) (width 0.15) (layer F.Cu) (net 1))
 (segment (start 97.85 82.043) (end 98.198 82.39099999999999) (width 0.15) (layer B.Cu) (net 1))
 (segment (start 98.198 82.39099999999999) (end 98.198 89.359) (width 0.15) (layer B.Cu) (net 1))
 (segment (start 98.198 89.359) (end 98.27846882023046 89.43946882023046) (width 0.15) (layer F.Cu) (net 1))
 (segment (start 98.27846882023046 89.43946882023046) (end 99.06177400000001 90.22277400000002) (width 0.15) (layer F.Cu) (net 1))
 (segment (start 99.06177400000001 90.22277400000002) (end 99.20368690909089 90.22277400000002) (width 0.15) (layer F.Cu) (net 1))
 (segment (start 105.56247890909097 87.67299600000007) (end 107.86196599999998 89.97296599999999) (width 0.15) (layer F.Cu) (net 1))
 (segment (start 107.86196599999998 89.97296599999999) (end 113.36231090909101 89.97296599999999) (width 0.15) (layer F.Cu) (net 1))
 (segment (start 110.96437019999988 101.33959600000009) (end 113.263566 103.639566) (width 0.15) (layer F.Cu) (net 1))
 (segment (start 113.263566 103.639566) (end 118.76420219999991 103.639566) (width 0.15) (layer F.Cu) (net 1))
 (segment (start 113.36231090909101 79.37303800000001) (end 113.36231090909101 79.373310909091) (width 0.15) (layer F.Cu) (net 1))
 (segment (start 113.36231090909101 79.373310909091) (end 113.36231090909101 89.97296599999999) (width 0.15) (layer F.Cu) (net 1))
 (segment (start 93.40006399999987 103.79984000000007) (end 90.60015999999993 103.79984000000007) (width 0.15) (layer F.Cu) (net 1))
 (segment (start 90.60015999999993 103.79984000000007) (end 84.34229399999987 110.05808433333361) (width 0.15) (layer F.Cu) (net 1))
 (segment (start 95.59618690909089 89.53277400000002) (end 97.24377400000002 89.53277400000002) (width 0.15) (layer F.Cu) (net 2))
 (segment (start 97.24377400000002 89.53277400000002) (end 97.93368690909088 90.22277400000002) (width 0.15) (layer F.Cu) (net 2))
 (segment (start 93.17618690909089 88.38027400000001) (end 92.02322599999998 89.53277400000002) (width 0.15) (layer F.Cu) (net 2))
 (segment (start 92.02322599999998 89.53277400000002) (end 90.75618690909089 89.53277400000002) (width 0.15) (layer F.Cu) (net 2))
 (segment (start 95.59618690909089 89.53277400000002) (end 94.32877400000001 89.53277400000002) (width 0.15) (layer F.Cu) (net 2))
 (segment (start 94.32877400000001 89.53277400000002) (end 93.17618690909089 88.38027400000001) (width 0.15) (layer F.Cu) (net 2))
 (segment (start 95.59618690909089 89.53277400000002) (end 94.7742449840031 89.53277400000002) (width 0.15) (layer F.Cu) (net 2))
 (segment (start 94.7742449840031 89.53277400000002) (end 94.6484023824909 89.40693139848781) (width 0.15) (layer F.Cu) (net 2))
 (segment (start 94.6484023824909 89.40693139848781) (end 94.63893139848781 89.40693139848781) (width 0.15) (layer F.Cu) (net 2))
 (segment (start 94.63893139848781 89.40693139848781) (end 94.617 89.385) (width 0.15) (layer F.Cu) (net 2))
 (segment (start 94.617 89.385) (end 95.6 88.402) (width 0.15) (layer B.Cu) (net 2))
 (segment (start 95.6 88.402) (end 95.6 86.29342593571471) (width 0.15) (layer B.Cu) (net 2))
 (segment (start 95.6 86.29342593571471) (end 95.6 86.123) (width 0.15) (layer B.Cu) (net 2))
 (segment (start 95.6 86.123) (end 95.6 86.669) (width 0.15) (layer F.Cu) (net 2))
 (segment (start 95.6 86.669) (end 95.59618690909089 86.67277400000002) (width 0.15) (layer F.Cu) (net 2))
 (segment (start 95.59618690909089 86.67277400000002) (end 95.59618690909089 85.26781309090912) (width 0.15) (layer F.Cu) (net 2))
 (segment (start 95.59618690909089 85.26781309090912) (end 97.11058690909073 83.75277400000002) (width 0.15) (layer F.Cu) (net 2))
 (segment (start 90.75618690909089 89.53277400000002) (end 89.17540600000002 91.11355490909088) (width 0.15) (layer F.Cu) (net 2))
 (segment (start 89.17540600000002 91.11355490909088) (end 89.17540600000002 94.10421433333335) (width 0.15) (layer F.Cu) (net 2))
 (segment (start 101.8999199999999 93.40006399999999) (end 99.42953215376764 90.92967615376773) (width 0.15) (layer F.Cu) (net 2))
 (segment (start 99.42953215376764 90.92967615376773) (end 98.6405890628586 90.92967615376773) (width 0.15) (layer F.Cu) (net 2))
 (segment (start 98.6405890628586 90.92967615376773) (end 97.93368690909088 90.22277400000002) (width 0.15) (layer F.Cu) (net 2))
 (segment (start 93.40006399999987 98.1000800000001) (end 93.1710800000001 98.1000800000001) (width 0.15) (layer F.Cu) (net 2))
 (segment (start 93.1710800000001 98.1000800000001) (end 89.17540600000002 94.10421433333335) (width 0.15) (layer F.Cu) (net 2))
 (segment (start 101.8999199999999 93.40006399999999) (end 101.8999199999999 92.84098274975041) (width 0.15) (layer F.Cu) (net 2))
 (segment (start 101.8999199999999 92.84098274975041) (end 102.38840285868287 92.35249989106744) (width 0.15) (layer F.Cu) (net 2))
 (segment (start 102.38840285868287 92.35249989106744) (end 102.38840285868287 92.21140285868287) (width 0.15) (layer F.Cu) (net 2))
 (segment (start 102.38840285868287 92.21140285868287) (end 102.355 92.178) (width 0.15) (layer F.Cu) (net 2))
 (segment (start 102.355 92.178) (end 102.355 89.286097196601) (width 0.15) (layer B.Cu) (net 2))
 (segment (start 102.355 89.286097196601) (end 102.9610467808358 88.68005041576521) (width 0.15) (layer B.Cu) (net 2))
 (segment (start 102.9610467808358 88.68005041576521) (end 102.9610467808358 88.6639532191642) (width 0.15) (layer B.Cu) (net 2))
 (segment (start 102.9610467808358 88.6639532191642) (end 103.091 88.534) (width 0.15) (layer B.Cu) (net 2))
 (segment (start 103.091 88.534) (end 103.091 87.67267513234043) (width 0.15) (layer F.Cu) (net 2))
 (segment (start 103.091 87.67267513234043) (end 104.2429014018625 86.52077373047793) (width 0.15) (layer F.Cu) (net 2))
 (segment (start 104.2429014018625 86.52077373047793) (end 104.71422626952207 86.52077373047793) (width 0.15) (layer F.Cu) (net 2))
 (segment (start 104.71422626952207 86.52077373047793) (end 105.56247890909097 85.67299999999994) (width 0.15) (layer F.Cu) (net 2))
 (segment (start 101.8999199999999 93.40006399999999) (end 101.8999199999999 94.3848789710923) (width 0.15) (layer F.Cu) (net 2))
 (segment (start 101.8999199999999 94.3848789710923) (end 103.6783556099343 96.16331458102671) (width 0.15) (layer F.Cu) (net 2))
 (segment (start 103.6783556099343 96.16331458102671) (end 103.6783556099343 96.1733556099343) (width 0.15) (layer F.Cu) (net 2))
 (segment (start 103.6783556099343 96.1733556099343) (end 103.8 96.295) (width 0.15) (layer F.Cu) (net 2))
 (segment (start 103.8 96.295) (end 107.162 96.295) (width 0.15) (layer B.Cu) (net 2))
 (segment (start 107.162 96.295) (end 108.65227396831156 97.78527396831156) (width 0.15) (layer B.Cu) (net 2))
 (segment (start 108.65227396831156 97.78527396831156) (end 108.712 97.845) (width 0.15) (layer B.Cu) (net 2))
 (segment (start 108.712 97.845) (end 110.207 99.34) (width 0.15) (layer F.Cu) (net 2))
 (segment (start 110.207 99.34) (end 110.96437019999988 99.33959999999996) (width 0.15) (layer F.Cu) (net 2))
 (gr_line (start 60 130) (end 140 130) (width 0.1) (layer Edge.Cuts))
 (gr_line (start 140 130) (end 140 70) (width 0.1) (layer Edge.Cuts))
 (gr_line (start 140 70) (end 60 70) (width 0.1) (layer Edge.Cuts))
 (gr_line (start 60 70) (end 60 130) (width 0.1) (layer Edge.Cuts))
 (via (at 103.537 82.574) (size 0.3) (drill 0.2) (layers F.Cu B.Cu) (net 6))
 (via (at 102.436 82.791) (size 0.3) (drill 0.2) (layers F.Cu B.Cu) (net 6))
 (via (at 100.6 83.928) (size 0.3) (drill 0.2) (layers F.Cu B.Cu) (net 6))
 (via (at 99.579 79.82300000000001) (size 0.3) (drill 0.2) (layers F.Cu B.Cu) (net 6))
 (via (at 107.846 95.276) (size 0.3) (drill 0.2) (layers F.Cu B.Cu) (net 6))
 (via (at 101 91) (size 0.3) (drill 0.2) (layers F.Cu B.Cu) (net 6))
 (via (at 94.347 89.871) (size 0.3) (drill 0.2) (layers F.Cu B.Cu) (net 1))
 (via (at 94.336 87.994) (size 0.3) (drill 0.2) (layers F.Cu B.Cu) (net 1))
 (via (at 104.421 92.129) (size 0.3) (drill 0.2) (layers F.Cu B.Cu) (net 1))
 (via (at 104.783 88.779) (size 0.3) (drill 0.2) (layers F.Cu B.Cu) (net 1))
 (via (at 97.85 82.043) (size 0.3) (drill 0.2) (layers F.Cu B.Cu) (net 1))
 (via (at 98.198 89.359) (size 0.3) (drill 0.2) (layers F.Cu B.Cu) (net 1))
 (via (at 94.617 89.385) (size 0.3) (drill 0.2) (layers F.Cu B.Cu) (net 2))
 (via (at 95.6 86.123) (size 0.3) (drill 0.2) (layers F.Cu B.Cu) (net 2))
 (via (at 102.355 92.178) (size 0.3) (drill 0.2) (layers F.Cu B.Cu) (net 2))
 (via (at 103.091 88.534) (size 0.3) (drill 0.2) (layers F.Cu B.Cu) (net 2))
 (via (at 103.8 96.295) (size 0.3) (drill 0.2) (layers F.Cu B.Cu) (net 2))
 (via (at 108.712 97.845) (size 0.3) (drill 0.2) (layers F.Cu B.Cu) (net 2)))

